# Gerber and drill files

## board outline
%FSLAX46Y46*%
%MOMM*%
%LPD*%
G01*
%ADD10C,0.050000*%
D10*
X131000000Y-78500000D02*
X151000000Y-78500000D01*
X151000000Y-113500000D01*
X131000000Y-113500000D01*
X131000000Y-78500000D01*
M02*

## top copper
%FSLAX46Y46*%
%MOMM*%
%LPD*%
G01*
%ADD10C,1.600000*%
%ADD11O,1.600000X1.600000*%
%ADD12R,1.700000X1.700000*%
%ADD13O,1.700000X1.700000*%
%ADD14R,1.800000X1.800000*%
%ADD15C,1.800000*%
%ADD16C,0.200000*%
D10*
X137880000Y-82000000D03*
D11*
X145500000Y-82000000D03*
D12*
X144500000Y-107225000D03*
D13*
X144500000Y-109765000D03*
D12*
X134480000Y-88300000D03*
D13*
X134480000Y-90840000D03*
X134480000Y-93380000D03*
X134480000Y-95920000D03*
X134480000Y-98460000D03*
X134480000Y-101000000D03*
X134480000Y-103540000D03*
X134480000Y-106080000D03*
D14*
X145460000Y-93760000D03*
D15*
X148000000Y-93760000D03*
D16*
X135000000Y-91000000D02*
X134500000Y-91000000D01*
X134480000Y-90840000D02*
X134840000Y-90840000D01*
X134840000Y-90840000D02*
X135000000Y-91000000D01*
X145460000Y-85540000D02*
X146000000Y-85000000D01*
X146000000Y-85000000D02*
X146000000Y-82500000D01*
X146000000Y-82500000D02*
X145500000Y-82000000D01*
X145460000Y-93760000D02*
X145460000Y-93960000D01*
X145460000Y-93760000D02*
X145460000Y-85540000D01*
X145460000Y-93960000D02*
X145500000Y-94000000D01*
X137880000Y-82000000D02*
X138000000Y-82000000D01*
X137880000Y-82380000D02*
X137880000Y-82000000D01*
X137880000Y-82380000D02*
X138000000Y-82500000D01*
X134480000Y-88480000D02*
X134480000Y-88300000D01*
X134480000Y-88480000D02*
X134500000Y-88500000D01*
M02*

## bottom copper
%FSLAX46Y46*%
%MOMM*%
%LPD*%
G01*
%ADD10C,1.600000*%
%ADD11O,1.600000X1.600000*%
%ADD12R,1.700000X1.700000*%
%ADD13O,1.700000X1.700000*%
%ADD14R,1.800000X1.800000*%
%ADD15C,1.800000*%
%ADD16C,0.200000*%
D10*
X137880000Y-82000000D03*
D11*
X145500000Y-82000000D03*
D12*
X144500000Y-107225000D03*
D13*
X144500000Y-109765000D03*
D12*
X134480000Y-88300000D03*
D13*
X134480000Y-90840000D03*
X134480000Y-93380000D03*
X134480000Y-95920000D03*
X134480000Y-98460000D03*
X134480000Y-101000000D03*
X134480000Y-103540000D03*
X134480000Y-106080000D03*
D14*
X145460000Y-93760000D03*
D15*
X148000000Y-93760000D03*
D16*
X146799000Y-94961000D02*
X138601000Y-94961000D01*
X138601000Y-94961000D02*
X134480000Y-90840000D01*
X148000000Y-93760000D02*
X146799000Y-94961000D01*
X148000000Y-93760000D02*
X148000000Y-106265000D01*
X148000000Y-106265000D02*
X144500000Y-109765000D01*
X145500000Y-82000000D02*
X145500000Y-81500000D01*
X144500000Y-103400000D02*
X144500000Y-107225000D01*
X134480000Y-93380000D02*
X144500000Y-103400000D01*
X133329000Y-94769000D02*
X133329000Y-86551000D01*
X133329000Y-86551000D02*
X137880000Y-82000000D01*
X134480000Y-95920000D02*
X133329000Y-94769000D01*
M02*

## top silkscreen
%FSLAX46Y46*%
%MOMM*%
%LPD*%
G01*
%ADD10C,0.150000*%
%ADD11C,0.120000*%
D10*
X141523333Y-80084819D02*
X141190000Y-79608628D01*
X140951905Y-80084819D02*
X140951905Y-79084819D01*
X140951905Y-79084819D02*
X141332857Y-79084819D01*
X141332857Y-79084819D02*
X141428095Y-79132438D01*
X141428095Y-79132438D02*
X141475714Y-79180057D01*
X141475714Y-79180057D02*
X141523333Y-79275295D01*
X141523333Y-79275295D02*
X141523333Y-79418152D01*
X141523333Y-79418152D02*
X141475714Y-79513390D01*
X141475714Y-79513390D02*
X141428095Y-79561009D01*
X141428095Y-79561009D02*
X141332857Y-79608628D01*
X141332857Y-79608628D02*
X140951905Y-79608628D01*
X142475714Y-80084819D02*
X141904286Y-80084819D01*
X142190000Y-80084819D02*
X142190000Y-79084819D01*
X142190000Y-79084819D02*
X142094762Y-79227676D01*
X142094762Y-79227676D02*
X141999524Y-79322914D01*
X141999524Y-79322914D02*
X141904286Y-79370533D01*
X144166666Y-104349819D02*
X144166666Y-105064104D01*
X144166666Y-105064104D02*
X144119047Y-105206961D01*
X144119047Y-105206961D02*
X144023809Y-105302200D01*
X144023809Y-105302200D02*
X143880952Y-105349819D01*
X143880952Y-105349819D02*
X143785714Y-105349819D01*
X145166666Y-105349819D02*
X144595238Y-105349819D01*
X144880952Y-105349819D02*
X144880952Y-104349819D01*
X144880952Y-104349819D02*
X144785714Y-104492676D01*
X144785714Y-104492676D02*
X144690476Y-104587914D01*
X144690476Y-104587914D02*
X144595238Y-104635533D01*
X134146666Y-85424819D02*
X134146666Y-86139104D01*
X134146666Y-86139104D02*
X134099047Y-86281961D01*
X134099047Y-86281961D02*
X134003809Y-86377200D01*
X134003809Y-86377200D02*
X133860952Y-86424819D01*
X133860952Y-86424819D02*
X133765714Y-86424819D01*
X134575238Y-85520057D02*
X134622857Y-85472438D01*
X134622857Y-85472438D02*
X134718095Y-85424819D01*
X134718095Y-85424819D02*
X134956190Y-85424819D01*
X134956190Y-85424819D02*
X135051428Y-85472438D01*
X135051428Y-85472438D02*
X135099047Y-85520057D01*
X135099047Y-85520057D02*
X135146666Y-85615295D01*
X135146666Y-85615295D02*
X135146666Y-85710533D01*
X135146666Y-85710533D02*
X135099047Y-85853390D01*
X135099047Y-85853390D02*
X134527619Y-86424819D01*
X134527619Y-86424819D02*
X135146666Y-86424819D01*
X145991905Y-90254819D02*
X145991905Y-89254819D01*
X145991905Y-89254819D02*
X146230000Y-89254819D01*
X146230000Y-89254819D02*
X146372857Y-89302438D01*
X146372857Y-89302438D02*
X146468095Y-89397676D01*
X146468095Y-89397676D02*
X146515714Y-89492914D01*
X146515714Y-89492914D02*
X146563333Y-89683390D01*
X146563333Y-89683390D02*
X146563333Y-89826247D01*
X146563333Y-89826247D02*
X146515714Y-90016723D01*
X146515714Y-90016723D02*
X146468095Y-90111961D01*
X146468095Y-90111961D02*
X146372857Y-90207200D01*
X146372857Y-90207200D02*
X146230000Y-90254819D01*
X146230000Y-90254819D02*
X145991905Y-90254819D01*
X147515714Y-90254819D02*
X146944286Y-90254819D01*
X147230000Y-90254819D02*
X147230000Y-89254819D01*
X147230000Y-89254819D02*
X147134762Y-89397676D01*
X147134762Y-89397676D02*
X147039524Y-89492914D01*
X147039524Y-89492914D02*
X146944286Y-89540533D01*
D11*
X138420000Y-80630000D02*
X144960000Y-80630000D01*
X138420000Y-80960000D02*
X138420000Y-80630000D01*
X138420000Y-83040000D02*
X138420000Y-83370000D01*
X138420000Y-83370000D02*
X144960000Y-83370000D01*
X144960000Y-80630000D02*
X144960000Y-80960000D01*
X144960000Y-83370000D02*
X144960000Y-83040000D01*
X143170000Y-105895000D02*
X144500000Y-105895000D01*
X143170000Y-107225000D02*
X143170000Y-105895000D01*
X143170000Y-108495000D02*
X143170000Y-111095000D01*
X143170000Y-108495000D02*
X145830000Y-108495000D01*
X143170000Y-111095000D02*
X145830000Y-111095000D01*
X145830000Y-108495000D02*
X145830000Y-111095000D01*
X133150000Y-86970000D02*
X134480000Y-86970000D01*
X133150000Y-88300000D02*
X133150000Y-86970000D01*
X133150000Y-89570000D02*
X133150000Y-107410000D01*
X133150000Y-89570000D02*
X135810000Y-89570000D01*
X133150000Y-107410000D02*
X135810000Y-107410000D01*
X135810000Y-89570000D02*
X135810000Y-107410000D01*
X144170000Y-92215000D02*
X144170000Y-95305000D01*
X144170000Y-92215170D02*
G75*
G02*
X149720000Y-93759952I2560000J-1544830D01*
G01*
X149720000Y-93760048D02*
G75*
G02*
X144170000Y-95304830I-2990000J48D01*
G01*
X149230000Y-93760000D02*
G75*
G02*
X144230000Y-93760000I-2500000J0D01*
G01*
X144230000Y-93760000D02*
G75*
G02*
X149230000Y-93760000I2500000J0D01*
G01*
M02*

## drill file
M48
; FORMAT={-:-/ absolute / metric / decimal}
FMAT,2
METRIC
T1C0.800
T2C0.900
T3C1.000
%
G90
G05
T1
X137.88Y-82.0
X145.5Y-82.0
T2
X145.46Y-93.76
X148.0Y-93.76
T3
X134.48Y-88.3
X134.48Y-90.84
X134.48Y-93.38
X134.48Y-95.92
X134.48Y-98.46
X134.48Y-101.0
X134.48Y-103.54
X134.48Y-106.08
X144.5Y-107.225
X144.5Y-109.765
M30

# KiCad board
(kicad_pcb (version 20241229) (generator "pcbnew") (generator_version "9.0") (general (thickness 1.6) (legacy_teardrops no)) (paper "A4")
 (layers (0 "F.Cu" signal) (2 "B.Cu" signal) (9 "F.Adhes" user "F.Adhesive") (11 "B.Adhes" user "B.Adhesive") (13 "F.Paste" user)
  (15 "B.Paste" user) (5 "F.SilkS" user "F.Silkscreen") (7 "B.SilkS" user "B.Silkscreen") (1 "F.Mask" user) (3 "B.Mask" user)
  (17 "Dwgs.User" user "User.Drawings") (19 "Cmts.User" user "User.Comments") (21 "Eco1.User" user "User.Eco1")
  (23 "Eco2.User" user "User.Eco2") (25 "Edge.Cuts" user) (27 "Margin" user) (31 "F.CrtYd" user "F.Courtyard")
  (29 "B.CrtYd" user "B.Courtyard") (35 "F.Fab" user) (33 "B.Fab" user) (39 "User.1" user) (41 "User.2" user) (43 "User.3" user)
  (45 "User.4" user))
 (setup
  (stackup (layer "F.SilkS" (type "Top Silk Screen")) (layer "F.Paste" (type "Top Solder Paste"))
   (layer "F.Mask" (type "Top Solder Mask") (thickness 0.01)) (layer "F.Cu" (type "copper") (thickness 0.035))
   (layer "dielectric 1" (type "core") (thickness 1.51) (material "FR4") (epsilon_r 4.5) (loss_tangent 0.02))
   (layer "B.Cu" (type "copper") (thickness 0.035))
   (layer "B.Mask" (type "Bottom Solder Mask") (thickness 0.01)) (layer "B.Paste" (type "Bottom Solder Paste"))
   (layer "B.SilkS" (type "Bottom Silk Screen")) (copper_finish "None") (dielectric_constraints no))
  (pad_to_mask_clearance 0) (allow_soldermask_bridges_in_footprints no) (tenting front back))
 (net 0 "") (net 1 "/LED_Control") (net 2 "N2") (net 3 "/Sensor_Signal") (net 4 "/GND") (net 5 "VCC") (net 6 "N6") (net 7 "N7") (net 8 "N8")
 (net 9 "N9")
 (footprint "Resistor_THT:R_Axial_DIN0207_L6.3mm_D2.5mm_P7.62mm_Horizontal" (layer "F.Cu") (at 137.88 82)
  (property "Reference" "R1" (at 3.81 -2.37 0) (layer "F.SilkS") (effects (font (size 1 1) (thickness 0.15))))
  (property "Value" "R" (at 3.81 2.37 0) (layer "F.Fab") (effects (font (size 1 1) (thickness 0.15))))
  (fp_line (start 0.54 -1.37) (end 7.08 -1.37) (stroke (width 0.12) (type solid)) (layer "F.SilkS"))
  (fp_line (start 0.54 -1.04) (end 0.54 -1.37) (stroke (width 0.12) (type solid)) (layer "F.SilkS"))
  (fp_line (start 0.54 1.04) (end 0.54 1.37) (stroke (width 0.12) (type solid)) (layer "F.SilkS"))
  (fp_line (start 0.54 1.37) (end 7.08 1.37) (stroke (width 0.12) (type solid)) (layer "F.SilkS"))
  (fp_line (start 7.08 -1.37) (end 7.08 -1.04) (stroke (width 0.12) (type solid)) (layer "F.SilkS"))
  (fp_line (start 7.08 1.37) (end 7.08 1.04) (stroke (width 0.12) (type solid)) (layer "F.SilkS"))
  (pad "1" thru_hole circle (at 0 0) (size 1.6 1.6) (drill 0.8) (layers "*.Cu" "*.Mask") (remove_unused_layers no) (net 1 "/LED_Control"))
  (pad "2" thru_hole oval (at 7.62 0) (size 1.6 1.6) (drill 0.8) (layers "*.Cu" "*.Mask") (remove_unused_layers no) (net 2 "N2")))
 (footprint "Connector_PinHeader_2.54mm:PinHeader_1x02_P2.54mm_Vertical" (layer "F.Cu") (at 144.5 107.225)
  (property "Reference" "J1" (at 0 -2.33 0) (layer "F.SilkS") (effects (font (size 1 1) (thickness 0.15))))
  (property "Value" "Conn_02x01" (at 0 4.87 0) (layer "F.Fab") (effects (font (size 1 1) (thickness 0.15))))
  (fp_line (start -1.33 -1.33) (end 0 -1.33) (stroke (width 0.12) (type solid)) (layer "F.SilkS"))
  (fp_line (start -1.33 0) (end -1.33 -1.33) (stroke (width 0.12) (type solid)) (layer "F.SilkS"))
  (fp_line (start -1.33 1.27) (end -1.33 3.87) (stroke (width 0.12) (type solid)) (layer "F.SilkS"))
  (fp_line (start -1.33 1.27) (end 1.33 1.27) (stroke (width 0.12) (type solid)) (layer "F.SilkS"))
  (fp_line (start -1.33 3.87) (end 1.33 3.87) (stroke (width 0.12) (type solid)) (layer "F.SilkS"))
  (fp_line (start 1.33 1.27) (end 1.33 3.87) (stroke (width 0.12) (type solid)) (layer "F.SilkS"))
  (pad "1" thru_hole rect (at 0 0) (size 1.7 1.7) (drill 1) (layers "*.Cu" "*.Mask") (remove_unused_layers no) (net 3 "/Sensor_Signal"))
  (pad "2" thru_hole oval (at 0 2.54) (size 1.7 1.7) (drill 1) (layers "*.Cu" "*.Mask") (remove_unused_layers no) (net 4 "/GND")))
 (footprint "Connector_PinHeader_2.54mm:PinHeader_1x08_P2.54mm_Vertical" (layer "F.Cu") (at 134.48 88.3)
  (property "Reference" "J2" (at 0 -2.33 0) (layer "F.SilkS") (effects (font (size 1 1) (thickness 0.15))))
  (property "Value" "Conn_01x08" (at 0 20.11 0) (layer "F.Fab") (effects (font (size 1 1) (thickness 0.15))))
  (fp_line (start -1.33 -1.33) (end 0 -1.33) (stroke (width 0.12) (type solid)) (layer "F.SilkS"))
  (fp_line (start -1.33 0) (end -1.33 -1.33) (stroke (width 0.12) (type solid)) (layer "F.SilkS"))
  (fp_line (start -1.33 1.27) (end -1.33 19.11) (stroke (width 0.12) (type solid)) (layer "F.SilkS"))
  (fp_line (start -1.33 1.27) (end 1.33 1.27) (stroke (width 0.12) (type solid)) (layer "F.SilkS"))
  (fp_line (start -1.33 19.11) (end 1.33 19.11) (stroke (width 0.12) (type solid)) (layer "F.SilkS"))
  (fp_line (start 1.33 1.27) (end 1.33 19.11) (stroke (width 0.12) (type solid)) (layer "F.SilkS"))
  (pad "1" thru_hole rect (at 0 0) (size 1.7 1.7) (drill 1) (layers "*.Cu" "*.Mask") (remove_unused_layers no) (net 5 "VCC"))
  (pad "2" thru_hole oval (at 0 2.54) (size 1.7 1.7) (drill 1) (layers "*.Cu" "*.Mask") (remove_unused_layers no) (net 4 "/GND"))
  (pad "3" thru_hole oval (at 0 5.08) (size 1.7 1.7) (drill 1) (layers "*.Cu" "*.Mask") (remove_unused_layers no) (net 3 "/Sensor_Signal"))
  (pad "4" thru_hole oval (at 0 7.62) (size 1.7 1.7) (drill 1) (layers "*.Cu" "*.Mask") (remove_unused_layers no) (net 1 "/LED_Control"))
  (pad "5" thru_hole oval (at 0 10.16) (size 1.7 1.7) (drill 1) (layers "*.Cu" "*.Mask") (remove_unused_layers no) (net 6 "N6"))
  (pad "6" thru_hole oval (at 0 12.7) (size 1.7 1.7) (drill 1) (layers "*.Cu" "*.Mask") (remove_unused_layers no) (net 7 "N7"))
  (pad "7" thru_hole oval (at 0 15.24) (size 1.7 1.7) (drill 1) (layers "*.Cu" "*.Mask") (remove_unused_layers no) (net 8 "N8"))
  (pad "8" thru_hole oval (at 0 17.78) (size 1.7 1.7) (drill 1) (layers "*.Cu" "*.Mask") (remove_unused_layers no) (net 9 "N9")))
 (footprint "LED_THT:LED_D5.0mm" (layer "F.Cu") (at 145.46 93.76)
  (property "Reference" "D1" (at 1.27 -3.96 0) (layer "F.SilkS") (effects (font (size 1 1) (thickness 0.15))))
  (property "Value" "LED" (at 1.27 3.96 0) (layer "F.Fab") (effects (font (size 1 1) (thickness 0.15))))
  (fp_line (start -1.29 -1.545) (end -1.29 1.545) (stroke (width 0.12) (type solid)) (layer "F.SilkS"))
  (fp_arc (start -1.29 -1.54483) (mid 2.071756 -2.880501) (end 4.26 -0.000048) (stroke (width 0.12) (type solid)) (layer "F.SilkS"))
  (fp_arc (start 4.26 0.000048) (mid 2.071756 2.880501) (end -1.29 1.54483) (stroke (width 0.12) (type solid)) (layer "F.SilkS"))
  (fp_circle (center 1.27 0) (end 3.77 0) (stroke (width 0.12) (type solid)) (fill no) (layer "F.SilkS"))
  (pad "1" thru_hole rect (at 0 0) (size 1.8 1.8) (drill 0.9) (layers "*.Cu" "*.Mask") (remove_unused_layers no) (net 2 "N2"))
  (pad "2" thru_hole circle (at 2.54 0) (size 1.8 1.8) (drill 0.9) (layers "*.Cu" "*.Mask") (remove_unused_layers no) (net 4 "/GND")))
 (gr_rect (start 131 78.5) (end 151 113.5) (stroke (width 0.05) (type default)) (fill no) (layer "Edge.Cuts"))
 (segment (start 135 91) (end 134.5 91) (width 0.2) (layer "F.Cu") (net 4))
 (segment (start 134.48 90.84) (end 134.84 90.84) (width 0.2) (layer "F.Cu") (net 4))
 (segment (start 134.84 90.84) (end 135 91) (width 0.2) (layer "F.Cu") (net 4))
 (segment (start 146.799 94.961) (end 138.601 94.961) (width 0.2) (layer "B.Cu") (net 4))
 (segment (start 138.601 94.961) (end 134.48 90.84) (width 0.2) (layer "B.Cu") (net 4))
 (segment (start 148 93.76) (end 146.799 94.961) (width 0.2) (layer "B.Cu") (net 4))
 (segment (start 148 93.76) (end 148 106.265) (width 0.2) (layer "B.Cu") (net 4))
 (segment (start 148 106.265) (end 144.5 109.765) (width 0.2) (layer "B.Cu") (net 4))
 (segment (start 145.46 85.54) (end 146 85) (width 0.2) (layer "F.Cu") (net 2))
 (segment (start 146 85) (end 146 82.5) (width 0.2) (layer "F.Cu") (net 2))
 (segment (start 146 82.5) (end 145.5 82) (width 0.2) (layer "F.Cu") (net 2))
 (segment (start 145.46 93.76) (end 145.46 93.96) (width 0.2) (layer "F.Cu") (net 2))
 (segment (start 145.46 93.76) (end 145.46 85.54) (width 0.2) (layer "F.Cu") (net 2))
 (segment (start 145.46 93.96) (end 145.5 94) (width 0.2) (layer "F.Cu") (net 2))
 (segment (start 145.5 82) (end 145.5 81.5) (width 0.2) (layer "B.Cu") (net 2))
 (segment (start 144.5 103.4) (end 144.5 107.225) (width 0.2) (layer "B.Cu") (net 3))
 (segment (start 134.48 93.38) (end 144.5 103.4) (width 0.2) (layer "B.Cu") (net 3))
 (segment (start 137.88 82) (end 138 82) (width 0.2) (layer "F.Cu") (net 1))
 (segment (start 137.88 82.38) (end 137.88 82) (width 0.2) (layer "F.Cu") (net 1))
 (segment (start 137.88 82.38) (end 138 82.5) (width 0.2) (layer "F.Cu") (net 1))
 (segment (start 133.329 94.769) (end 133.329 86.551) (width 0.2) (layer "B.Cu") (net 1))
 (segment (start 133.329 86.551) (end 137.88 82) (width 0.2) (layer "B.Cu") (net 1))
 (segment (start 134.48 95.92) (end 133.329 94.769) (width 0.2) (layer "B.Cu") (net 1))
 (segment (start 134.48 88.48) (end 134.48 88.3) (width 0.2) (layer "F.Cu") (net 5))
 (segment (start 134.48 88.48) (end 134.5 88.5) (width 0.2) (layer "F.Cu") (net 5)))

